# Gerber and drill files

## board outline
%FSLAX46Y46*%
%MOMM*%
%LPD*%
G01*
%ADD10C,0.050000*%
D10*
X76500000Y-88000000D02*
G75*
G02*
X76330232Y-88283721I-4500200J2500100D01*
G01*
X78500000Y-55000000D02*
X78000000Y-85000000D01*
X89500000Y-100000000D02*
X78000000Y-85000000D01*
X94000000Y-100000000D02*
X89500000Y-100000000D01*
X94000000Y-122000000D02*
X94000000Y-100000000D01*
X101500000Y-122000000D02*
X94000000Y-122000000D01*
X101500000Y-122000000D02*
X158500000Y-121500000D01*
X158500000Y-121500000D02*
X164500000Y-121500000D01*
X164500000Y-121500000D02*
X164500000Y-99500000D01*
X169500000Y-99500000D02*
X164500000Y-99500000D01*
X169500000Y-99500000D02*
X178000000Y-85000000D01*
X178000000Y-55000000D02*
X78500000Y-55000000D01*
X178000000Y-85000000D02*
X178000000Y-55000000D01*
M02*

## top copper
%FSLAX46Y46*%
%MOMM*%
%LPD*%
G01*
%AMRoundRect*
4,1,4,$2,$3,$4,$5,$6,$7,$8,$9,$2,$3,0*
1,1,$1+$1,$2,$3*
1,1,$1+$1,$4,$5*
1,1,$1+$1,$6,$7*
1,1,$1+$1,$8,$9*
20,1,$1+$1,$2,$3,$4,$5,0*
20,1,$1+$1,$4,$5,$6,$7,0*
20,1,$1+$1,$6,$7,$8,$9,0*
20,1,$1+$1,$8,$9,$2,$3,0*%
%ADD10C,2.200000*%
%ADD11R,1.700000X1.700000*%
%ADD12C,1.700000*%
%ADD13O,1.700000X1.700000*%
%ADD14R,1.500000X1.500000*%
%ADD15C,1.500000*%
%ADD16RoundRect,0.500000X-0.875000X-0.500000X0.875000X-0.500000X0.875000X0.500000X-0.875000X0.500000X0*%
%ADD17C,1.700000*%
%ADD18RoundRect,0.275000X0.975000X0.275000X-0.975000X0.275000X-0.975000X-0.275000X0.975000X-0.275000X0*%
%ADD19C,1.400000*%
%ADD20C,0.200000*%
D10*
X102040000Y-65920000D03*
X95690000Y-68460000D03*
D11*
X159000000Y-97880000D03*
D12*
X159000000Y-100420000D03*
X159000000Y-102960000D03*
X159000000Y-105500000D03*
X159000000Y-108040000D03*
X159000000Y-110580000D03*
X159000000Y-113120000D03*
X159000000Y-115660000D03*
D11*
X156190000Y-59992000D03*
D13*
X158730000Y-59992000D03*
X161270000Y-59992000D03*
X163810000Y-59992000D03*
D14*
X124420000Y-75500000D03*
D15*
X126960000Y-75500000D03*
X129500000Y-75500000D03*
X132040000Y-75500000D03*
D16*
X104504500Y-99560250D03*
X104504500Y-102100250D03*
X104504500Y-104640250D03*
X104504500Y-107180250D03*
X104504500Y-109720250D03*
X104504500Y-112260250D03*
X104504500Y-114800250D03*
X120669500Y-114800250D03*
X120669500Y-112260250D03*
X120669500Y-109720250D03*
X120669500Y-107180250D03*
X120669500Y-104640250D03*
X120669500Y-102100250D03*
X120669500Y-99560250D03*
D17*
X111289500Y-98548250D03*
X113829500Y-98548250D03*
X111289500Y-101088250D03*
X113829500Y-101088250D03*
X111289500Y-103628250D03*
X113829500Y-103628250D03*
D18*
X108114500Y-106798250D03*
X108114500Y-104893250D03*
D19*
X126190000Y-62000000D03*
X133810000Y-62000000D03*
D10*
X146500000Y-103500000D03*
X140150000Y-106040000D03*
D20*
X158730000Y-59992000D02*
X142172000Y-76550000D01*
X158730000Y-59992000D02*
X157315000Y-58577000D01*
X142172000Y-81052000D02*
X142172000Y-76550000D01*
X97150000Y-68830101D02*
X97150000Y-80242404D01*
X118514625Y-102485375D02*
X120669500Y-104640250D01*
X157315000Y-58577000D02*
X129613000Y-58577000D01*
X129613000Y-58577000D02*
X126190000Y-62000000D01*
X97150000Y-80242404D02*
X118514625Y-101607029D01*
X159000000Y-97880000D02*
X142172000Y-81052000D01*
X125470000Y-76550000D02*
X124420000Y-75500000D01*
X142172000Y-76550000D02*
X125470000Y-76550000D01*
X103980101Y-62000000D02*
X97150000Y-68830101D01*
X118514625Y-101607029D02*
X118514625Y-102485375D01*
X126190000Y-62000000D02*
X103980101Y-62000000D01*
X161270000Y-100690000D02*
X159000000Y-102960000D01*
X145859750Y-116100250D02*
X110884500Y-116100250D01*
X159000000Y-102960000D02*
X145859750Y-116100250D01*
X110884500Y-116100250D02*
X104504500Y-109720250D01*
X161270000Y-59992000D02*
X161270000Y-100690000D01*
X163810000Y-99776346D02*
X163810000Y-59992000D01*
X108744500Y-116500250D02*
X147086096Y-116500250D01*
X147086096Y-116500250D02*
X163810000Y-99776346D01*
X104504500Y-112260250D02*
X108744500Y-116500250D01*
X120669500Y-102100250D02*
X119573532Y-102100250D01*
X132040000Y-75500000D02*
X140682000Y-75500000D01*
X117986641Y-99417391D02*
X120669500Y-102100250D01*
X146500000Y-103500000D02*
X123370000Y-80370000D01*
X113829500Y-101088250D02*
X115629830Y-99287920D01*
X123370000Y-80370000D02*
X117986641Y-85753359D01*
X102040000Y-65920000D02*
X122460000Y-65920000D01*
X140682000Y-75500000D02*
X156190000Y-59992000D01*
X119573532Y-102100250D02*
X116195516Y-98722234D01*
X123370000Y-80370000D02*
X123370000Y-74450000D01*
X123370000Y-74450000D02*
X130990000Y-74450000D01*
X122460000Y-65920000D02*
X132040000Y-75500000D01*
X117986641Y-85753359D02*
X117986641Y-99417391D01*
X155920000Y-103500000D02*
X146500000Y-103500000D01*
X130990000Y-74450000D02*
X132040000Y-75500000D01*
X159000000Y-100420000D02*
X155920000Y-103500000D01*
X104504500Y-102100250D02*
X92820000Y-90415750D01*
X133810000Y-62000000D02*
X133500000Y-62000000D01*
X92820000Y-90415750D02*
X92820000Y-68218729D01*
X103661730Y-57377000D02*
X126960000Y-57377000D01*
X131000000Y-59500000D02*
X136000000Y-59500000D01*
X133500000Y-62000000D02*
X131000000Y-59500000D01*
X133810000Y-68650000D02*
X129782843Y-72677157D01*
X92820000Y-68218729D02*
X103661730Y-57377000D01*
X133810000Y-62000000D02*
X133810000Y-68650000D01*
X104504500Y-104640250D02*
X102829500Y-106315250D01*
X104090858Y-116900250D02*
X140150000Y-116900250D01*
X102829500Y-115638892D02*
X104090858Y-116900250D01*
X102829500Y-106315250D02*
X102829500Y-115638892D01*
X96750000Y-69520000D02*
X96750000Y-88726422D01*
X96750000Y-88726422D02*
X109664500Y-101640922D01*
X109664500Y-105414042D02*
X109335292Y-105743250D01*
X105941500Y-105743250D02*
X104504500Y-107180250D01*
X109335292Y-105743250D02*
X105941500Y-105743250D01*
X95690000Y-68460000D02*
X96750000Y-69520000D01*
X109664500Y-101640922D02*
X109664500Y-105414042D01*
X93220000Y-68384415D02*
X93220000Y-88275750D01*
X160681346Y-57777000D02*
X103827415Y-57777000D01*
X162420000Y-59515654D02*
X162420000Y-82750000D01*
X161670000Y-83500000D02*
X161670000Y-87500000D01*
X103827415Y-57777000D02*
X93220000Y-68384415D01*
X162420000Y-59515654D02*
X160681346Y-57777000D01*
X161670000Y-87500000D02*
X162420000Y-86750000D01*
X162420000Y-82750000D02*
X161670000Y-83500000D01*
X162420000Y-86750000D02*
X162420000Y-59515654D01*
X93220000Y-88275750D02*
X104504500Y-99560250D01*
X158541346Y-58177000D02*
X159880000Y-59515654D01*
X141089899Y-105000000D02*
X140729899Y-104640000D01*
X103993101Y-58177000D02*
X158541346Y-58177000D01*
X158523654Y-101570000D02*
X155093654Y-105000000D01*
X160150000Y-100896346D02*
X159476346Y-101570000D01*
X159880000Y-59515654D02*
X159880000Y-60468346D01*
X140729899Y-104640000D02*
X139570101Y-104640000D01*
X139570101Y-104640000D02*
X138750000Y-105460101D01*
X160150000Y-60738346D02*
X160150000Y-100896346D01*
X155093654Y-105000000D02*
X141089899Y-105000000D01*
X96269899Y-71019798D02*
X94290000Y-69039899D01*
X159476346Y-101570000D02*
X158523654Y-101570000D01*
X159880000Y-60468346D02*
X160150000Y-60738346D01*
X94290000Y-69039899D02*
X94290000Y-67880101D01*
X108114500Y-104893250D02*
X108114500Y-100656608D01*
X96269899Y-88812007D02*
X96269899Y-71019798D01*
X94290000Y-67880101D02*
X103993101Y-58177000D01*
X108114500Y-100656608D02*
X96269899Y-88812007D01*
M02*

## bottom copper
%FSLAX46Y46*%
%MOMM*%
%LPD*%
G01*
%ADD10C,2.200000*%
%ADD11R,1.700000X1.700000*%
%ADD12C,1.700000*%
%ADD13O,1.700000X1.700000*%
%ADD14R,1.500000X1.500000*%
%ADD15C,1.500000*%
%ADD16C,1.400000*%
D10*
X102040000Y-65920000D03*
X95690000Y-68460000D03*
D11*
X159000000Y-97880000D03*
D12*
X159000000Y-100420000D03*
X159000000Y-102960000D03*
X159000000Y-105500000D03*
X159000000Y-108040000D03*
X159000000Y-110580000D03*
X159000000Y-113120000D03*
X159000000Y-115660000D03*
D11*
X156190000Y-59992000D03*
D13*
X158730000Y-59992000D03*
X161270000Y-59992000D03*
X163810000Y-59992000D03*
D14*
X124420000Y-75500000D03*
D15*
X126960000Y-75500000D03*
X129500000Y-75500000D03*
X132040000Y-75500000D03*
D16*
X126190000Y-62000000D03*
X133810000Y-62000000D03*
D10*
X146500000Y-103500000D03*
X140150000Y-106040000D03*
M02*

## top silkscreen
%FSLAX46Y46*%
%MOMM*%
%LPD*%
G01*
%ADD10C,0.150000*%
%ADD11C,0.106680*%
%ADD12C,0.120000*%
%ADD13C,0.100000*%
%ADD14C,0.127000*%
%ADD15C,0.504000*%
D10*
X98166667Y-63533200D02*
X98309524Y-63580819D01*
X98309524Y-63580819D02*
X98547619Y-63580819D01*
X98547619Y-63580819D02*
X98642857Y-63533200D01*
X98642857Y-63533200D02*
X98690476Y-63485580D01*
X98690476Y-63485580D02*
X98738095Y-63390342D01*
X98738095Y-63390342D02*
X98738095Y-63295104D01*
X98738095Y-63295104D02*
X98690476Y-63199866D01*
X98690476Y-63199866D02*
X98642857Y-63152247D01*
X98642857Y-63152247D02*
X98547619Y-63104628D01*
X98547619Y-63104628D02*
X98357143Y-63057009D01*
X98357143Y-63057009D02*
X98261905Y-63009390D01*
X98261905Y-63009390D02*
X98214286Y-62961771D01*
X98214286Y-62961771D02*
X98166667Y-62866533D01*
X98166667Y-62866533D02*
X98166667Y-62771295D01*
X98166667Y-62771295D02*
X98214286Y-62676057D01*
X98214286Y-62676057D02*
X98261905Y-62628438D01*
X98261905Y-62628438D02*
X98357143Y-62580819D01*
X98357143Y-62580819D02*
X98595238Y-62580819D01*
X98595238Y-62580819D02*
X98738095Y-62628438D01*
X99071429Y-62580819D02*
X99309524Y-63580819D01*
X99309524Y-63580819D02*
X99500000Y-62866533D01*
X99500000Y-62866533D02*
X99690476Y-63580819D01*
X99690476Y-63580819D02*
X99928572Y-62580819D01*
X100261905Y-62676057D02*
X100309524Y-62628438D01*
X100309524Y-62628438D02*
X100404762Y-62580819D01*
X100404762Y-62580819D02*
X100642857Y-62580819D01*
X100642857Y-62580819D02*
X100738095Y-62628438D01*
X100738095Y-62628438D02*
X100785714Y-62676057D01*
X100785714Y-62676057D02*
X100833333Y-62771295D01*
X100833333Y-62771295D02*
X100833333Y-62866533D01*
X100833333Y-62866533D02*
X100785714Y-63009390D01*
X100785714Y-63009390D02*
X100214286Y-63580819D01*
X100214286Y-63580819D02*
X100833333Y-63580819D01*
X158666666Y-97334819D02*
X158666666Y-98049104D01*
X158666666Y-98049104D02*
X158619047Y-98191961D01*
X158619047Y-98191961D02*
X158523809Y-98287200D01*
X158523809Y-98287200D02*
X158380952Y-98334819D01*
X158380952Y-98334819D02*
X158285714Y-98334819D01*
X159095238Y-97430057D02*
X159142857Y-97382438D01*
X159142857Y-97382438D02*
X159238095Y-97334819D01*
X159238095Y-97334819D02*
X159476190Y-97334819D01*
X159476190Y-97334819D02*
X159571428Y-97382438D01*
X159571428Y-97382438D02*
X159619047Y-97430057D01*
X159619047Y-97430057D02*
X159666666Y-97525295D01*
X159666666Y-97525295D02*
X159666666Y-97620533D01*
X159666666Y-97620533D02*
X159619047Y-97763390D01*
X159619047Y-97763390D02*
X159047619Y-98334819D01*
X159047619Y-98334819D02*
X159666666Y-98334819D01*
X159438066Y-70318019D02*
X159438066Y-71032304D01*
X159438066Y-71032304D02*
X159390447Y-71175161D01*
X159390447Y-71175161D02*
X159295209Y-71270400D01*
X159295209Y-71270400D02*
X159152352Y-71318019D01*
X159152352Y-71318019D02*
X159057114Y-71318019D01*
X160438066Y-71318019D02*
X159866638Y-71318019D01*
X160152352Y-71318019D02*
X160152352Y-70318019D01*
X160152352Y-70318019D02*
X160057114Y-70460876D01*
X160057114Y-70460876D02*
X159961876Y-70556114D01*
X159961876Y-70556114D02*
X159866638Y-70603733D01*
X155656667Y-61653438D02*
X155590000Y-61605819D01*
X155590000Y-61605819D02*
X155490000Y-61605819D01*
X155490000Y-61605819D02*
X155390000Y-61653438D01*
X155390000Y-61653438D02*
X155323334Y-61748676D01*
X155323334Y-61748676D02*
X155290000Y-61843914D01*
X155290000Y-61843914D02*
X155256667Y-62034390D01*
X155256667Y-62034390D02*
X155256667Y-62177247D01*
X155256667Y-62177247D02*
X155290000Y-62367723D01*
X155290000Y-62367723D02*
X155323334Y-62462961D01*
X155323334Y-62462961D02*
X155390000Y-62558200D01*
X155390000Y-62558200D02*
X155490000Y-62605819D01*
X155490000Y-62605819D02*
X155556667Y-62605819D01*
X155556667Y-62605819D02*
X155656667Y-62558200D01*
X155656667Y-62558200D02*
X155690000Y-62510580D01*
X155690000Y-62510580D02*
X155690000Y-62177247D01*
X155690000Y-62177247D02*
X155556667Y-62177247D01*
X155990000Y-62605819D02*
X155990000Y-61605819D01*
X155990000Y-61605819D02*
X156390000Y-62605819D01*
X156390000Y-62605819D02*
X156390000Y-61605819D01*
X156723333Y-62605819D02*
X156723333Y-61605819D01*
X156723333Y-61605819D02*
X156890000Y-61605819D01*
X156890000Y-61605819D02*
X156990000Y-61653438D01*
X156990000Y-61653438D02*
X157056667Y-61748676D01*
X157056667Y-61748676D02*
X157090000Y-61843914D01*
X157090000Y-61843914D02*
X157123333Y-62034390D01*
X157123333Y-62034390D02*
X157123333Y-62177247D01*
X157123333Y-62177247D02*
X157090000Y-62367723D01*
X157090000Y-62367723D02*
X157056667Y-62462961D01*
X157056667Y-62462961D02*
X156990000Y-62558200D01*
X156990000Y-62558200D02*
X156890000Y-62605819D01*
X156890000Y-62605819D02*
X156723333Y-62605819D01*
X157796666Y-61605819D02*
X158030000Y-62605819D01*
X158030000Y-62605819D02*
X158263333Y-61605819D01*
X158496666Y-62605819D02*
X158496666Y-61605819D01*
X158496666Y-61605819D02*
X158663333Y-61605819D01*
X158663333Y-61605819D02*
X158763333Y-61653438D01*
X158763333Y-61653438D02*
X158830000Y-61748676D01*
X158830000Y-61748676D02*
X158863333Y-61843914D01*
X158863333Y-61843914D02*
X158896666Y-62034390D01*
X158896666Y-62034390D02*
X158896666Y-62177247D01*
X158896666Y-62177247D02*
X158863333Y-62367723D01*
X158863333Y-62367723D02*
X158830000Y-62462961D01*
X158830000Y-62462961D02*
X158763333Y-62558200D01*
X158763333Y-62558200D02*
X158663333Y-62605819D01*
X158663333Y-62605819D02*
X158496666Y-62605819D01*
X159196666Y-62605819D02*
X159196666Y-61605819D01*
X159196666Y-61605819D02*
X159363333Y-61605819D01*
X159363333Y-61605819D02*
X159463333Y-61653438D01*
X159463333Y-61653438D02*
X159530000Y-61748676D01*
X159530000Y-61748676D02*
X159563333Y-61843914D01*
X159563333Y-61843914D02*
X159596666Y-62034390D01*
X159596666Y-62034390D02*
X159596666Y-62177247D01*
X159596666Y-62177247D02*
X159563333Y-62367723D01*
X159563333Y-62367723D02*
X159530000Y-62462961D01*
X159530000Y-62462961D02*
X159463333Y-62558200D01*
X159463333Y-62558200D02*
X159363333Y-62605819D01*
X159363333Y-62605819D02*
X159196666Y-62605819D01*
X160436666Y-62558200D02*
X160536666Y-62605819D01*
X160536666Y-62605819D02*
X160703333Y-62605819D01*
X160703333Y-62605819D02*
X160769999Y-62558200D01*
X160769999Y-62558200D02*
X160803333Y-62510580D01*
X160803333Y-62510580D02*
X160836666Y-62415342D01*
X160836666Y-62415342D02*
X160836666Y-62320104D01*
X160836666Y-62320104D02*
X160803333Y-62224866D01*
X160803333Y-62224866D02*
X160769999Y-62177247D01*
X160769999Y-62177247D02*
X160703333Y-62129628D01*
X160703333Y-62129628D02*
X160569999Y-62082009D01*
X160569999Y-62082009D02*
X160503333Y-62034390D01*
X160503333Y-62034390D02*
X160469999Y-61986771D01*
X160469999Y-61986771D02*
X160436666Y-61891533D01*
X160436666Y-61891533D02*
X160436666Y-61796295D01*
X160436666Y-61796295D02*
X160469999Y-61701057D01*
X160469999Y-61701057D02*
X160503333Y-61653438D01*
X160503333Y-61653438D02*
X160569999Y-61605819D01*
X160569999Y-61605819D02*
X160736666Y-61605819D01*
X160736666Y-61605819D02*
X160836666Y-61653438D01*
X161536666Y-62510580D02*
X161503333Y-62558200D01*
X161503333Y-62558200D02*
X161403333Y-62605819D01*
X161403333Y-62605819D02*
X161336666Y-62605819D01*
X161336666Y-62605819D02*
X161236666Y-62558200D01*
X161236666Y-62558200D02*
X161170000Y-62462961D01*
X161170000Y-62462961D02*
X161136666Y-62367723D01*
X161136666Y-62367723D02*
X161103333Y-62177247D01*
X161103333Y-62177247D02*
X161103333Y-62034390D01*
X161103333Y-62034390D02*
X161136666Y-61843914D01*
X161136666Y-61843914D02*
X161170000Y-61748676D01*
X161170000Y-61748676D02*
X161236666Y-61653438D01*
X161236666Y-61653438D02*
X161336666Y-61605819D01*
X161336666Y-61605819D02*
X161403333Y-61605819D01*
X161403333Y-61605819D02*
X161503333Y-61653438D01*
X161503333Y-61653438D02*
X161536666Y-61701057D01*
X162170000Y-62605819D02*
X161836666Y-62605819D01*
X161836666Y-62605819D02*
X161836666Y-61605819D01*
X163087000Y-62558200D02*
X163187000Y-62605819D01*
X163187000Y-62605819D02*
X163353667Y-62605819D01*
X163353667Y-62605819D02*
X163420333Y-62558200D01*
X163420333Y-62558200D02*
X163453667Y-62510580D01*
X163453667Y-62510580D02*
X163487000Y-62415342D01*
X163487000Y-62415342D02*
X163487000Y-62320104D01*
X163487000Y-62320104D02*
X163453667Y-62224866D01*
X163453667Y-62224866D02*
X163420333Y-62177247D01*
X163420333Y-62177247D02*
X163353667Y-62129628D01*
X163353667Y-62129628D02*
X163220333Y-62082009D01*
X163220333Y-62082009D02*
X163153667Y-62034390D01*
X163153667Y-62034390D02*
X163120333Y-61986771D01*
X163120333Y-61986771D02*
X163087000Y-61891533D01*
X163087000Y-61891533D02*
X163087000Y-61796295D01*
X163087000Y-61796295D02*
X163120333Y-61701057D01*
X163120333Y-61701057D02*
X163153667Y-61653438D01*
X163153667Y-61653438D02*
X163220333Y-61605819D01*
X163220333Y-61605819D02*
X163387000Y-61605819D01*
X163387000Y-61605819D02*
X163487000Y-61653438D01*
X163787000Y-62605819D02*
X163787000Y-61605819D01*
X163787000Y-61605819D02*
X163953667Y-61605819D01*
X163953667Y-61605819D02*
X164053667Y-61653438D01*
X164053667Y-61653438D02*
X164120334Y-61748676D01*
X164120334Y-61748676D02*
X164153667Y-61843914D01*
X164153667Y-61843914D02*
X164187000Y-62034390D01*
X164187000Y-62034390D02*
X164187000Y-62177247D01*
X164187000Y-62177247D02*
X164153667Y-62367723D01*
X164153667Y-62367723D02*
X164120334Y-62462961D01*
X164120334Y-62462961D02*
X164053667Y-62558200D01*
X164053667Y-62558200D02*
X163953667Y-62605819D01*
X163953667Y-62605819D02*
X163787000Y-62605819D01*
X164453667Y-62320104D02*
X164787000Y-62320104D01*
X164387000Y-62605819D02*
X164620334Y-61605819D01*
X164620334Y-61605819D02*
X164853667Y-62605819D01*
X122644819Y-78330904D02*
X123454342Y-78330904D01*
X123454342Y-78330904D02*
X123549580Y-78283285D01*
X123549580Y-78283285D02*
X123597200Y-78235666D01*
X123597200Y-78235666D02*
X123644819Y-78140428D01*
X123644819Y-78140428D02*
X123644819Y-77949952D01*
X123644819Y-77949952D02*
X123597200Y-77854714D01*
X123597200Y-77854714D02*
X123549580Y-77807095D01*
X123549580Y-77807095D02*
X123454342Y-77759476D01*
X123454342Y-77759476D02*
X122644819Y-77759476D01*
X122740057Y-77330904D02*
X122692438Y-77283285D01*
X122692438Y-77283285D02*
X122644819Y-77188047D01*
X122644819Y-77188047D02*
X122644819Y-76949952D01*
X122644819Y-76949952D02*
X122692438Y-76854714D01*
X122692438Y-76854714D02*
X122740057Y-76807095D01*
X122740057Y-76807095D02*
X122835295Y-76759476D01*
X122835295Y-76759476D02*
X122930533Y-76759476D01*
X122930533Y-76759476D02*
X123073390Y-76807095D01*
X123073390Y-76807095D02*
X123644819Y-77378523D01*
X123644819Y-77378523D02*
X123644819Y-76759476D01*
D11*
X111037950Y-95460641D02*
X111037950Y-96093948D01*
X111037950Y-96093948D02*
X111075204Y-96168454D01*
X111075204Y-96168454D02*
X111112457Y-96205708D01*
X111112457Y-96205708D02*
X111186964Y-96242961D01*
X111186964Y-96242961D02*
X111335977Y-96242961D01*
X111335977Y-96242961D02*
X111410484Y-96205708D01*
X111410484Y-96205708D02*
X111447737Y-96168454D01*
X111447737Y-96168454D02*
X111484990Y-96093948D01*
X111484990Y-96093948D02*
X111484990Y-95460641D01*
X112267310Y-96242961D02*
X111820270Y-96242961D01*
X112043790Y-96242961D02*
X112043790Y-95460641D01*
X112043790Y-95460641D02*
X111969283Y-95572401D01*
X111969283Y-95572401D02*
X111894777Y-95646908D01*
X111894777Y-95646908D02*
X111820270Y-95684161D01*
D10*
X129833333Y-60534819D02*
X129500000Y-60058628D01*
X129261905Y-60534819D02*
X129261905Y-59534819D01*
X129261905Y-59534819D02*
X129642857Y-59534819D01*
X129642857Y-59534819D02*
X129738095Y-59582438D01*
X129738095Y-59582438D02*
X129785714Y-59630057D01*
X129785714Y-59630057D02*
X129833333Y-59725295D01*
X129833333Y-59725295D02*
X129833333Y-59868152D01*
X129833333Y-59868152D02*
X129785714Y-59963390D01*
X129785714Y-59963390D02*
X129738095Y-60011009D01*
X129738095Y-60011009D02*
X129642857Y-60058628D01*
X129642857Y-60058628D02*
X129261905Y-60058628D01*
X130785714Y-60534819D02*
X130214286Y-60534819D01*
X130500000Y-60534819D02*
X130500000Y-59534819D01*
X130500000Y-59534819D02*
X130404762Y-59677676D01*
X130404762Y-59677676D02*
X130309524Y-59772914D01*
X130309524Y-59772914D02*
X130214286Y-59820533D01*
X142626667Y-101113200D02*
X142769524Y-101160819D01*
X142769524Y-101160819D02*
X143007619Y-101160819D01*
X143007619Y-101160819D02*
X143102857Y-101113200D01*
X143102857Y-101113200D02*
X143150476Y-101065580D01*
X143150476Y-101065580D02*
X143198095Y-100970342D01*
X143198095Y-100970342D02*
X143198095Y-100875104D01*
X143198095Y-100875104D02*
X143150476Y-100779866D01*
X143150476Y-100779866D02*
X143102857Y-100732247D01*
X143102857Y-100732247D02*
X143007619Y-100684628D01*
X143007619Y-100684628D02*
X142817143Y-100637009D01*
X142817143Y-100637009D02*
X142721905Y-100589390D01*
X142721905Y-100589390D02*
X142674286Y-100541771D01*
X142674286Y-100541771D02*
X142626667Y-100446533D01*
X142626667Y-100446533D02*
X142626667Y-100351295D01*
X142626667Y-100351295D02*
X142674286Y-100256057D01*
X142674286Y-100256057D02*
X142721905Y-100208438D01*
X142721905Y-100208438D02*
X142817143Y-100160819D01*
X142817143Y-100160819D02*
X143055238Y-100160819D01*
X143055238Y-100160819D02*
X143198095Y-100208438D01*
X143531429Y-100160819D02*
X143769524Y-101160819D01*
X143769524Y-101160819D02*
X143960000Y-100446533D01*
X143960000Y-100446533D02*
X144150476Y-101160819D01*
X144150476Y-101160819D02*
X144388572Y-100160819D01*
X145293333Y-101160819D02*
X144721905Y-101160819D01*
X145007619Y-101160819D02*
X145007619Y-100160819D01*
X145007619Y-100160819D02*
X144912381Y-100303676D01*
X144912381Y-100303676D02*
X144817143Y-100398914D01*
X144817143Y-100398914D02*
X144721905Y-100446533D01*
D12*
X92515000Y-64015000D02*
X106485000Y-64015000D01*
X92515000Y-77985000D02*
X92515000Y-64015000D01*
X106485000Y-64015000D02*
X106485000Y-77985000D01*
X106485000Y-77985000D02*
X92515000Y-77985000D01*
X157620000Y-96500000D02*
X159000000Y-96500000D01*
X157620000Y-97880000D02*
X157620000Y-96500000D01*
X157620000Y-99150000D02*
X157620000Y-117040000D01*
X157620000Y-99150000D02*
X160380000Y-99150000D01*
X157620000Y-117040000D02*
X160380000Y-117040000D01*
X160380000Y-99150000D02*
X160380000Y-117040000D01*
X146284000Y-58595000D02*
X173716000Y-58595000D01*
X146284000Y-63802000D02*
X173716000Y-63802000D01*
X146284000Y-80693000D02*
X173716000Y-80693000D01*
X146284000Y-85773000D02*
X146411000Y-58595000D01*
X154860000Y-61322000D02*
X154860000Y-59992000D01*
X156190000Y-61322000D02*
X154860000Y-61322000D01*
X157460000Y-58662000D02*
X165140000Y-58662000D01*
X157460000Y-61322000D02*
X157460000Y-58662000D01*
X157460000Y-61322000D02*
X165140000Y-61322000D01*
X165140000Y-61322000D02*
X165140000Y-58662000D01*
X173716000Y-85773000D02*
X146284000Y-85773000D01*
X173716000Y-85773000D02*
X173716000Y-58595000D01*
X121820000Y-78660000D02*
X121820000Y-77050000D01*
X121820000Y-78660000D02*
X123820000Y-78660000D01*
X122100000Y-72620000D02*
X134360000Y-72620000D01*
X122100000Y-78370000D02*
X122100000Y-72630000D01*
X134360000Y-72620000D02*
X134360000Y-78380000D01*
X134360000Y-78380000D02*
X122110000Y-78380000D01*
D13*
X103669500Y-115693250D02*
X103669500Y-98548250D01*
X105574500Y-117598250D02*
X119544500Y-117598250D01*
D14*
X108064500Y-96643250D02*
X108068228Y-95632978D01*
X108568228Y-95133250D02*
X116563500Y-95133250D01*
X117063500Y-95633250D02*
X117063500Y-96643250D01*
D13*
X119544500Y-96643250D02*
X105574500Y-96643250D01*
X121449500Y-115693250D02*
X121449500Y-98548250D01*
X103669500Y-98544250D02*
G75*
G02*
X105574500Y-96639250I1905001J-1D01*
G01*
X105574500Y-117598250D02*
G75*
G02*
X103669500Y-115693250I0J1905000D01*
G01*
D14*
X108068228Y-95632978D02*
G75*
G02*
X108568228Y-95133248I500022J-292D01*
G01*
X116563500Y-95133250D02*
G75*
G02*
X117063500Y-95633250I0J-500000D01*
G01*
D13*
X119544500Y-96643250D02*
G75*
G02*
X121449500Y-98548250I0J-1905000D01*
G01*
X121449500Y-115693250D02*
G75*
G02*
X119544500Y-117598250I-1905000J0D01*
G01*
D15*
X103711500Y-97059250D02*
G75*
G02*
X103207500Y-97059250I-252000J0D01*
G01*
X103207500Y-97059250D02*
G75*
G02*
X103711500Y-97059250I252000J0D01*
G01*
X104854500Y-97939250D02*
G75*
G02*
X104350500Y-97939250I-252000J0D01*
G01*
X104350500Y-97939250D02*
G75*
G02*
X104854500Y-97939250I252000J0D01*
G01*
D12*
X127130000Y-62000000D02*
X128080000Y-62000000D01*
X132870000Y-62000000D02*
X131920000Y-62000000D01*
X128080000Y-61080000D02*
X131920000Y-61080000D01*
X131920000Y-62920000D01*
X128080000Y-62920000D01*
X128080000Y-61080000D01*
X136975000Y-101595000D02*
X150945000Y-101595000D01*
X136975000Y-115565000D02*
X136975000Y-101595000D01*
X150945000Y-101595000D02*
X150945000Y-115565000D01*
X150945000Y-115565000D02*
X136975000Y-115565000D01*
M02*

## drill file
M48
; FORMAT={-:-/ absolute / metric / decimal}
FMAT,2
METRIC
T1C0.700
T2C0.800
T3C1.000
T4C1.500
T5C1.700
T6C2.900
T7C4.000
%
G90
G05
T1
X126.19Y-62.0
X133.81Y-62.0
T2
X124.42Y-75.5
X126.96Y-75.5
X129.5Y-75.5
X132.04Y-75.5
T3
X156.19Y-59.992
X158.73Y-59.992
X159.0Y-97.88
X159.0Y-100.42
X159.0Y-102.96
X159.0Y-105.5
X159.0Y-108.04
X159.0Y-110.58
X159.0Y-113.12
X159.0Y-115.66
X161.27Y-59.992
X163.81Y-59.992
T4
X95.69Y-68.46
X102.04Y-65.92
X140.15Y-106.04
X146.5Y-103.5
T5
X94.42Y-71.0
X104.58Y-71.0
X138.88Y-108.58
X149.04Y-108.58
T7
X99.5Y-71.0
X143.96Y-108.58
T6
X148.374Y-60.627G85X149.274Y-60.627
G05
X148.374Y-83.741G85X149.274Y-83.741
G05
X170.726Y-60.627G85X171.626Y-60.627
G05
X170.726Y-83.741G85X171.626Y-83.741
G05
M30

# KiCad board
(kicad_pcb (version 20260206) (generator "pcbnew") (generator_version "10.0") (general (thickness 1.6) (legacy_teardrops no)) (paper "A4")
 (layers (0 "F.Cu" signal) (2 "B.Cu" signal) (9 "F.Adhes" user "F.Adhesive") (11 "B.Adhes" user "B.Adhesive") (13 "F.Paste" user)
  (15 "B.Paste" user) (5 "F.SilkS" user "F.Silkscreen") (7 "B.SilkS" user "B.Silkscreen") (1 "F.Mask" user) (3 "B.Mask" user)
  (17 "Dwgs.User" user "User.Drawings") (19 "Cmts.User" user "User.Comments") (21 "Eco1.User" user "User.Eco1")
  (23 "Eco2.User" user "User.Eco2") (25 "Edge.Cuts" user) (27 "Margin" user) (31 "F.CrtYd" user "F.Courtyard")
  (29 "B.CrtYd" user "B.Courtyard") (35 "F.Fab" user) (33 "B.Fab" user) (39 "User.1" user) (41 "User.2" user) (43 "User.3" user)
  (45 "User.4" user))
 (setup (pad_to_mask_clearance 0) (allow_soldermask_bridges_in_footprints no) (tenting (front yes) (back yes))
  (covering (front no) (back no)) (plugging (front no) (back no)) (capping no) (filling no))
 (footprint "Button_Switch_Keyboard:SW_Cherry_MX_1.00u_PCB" (layer "F.Cu") (at 102.04 65.92)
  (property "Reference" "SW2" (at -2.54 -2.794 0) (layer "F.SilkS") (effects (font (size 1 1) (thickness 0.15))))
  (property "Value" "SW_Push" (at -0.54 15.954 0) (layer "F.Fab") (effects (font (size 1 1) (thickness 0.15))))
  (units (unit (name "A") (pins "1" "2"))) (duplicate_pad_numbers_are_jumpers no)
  (fp_line (start -9.525 -1.905) (end 4.445 -1.905) (stroke (width 0.12) (type solid)) (layer "F.SilkS"))
  (fp_line (start -9.525 12.065) (end -9.525 -1.905) (stroke (width 0.12) (type solid)) (layer "F.SilkS"))
  (fp_line (start 4.445 -1.905) (end 4.445 12.065) (stroke (width 0.12) (type solid)) (layer "F.SilkS"))
  (fp_line (start 4.445 12.065) (end -9.525 12.065) (stroke (width 0.12) (type solid)) (layer "F.SilkS"))
  (pad "" np_thru_hole circle (at -7.62 5.08) (size 1.7 1.7) (drill 1.7) (layers "*.Cu" "*.Mask"))
  (pad "" np_thru_hole circle (at -2.54 5.08) (size 4 4) (drill 4) (layers "*.Cu" "*.Mask"))
  (pad "" np_thru_hole circle (at 2.54 5.08) (size 1.7 1.7) (drill 1.7) (layers "*.Cu" "*.Mask"))
  (pad "1" thru_hole circle (at 0 0) (size 2.2 2.2) (drill 1.5) (layers "*.Cu" "*.Mask") (remove_unused_layers no) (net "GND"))
  (pad "2" thru_hole circle (at -6.35 2.54) (size 2.2 2.2) (drill 1.5) (layers "*.Cu" "*.Mask") (remove_unused_layers no) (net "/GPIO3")))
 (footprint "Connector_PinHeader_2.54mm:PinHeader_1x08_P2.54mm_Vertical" (layer "F.Cu") (at 159 97.88)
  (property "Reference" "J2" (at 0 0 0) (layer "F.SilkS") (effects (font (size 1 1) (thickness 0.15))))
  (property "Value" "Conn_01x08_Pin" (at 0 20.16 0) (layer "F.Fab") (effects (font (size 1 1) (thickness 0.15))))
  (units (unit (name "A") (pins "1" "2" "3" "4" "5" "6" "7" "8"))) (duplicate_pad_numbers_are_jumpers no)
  (fp_line (start -1.38 -1.38) (end 0 -1.38) (stroke (width 0.12) (type solid)) (layer "F.SilkS"))
  (fp_line (start -1.38 0) (end -1.38 -1.38) (stroke (width 0.12) (type solid)) (layer "F.SilkS"))
  (fp_line (start -1.38 1.27) (end -1.38 19.16) (stroke (width 0.12) (type solid)) (layer "F.SilkS"))
  (fp_line (start -1.38 1.27) (end 1.38 1.27) (stroke (width 0.12) (type solid)) (layer "F.SilkS"))
  (fp_line (start -1.38 19.16) (end 1.38 19.16) (stroke (width 0.12) (type solid)) (layer "F.SilkS"))
  (fp_line (start 1.38 1.27) (end 1.38 19.16) (stroke (width 0.12) (type solid)) (layer "F.SilkS"))
  (pad "1" thru_hole rect (at 0 0) (size 1.7 1.7) (drill 1) (layers "*.Cu" "*.Mask") (remove_unused_layers no) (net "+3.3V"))
  (pad "2" thru_hole circle (at 0 2.54) (size 1.7 1.7) (drill 1) (layers "*.Cu" "*.Mask") (remove_unused_layers no) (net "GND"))
  (pad "3" thru_hole circle (at 0 5.08) (size 1.7 1.7) (drill 1) (layers "*.Cu" "*.Mask") (remove_unused_layers no) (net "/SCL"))
  (pad "4" thru_hole circle (at 0 7.62) (size 1.7 1.7) (drill 1) (layers "*.Cu" "*.Mask") (remove_unused_layers no) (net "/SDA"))
  (pad "5" thru_hole circle (at 0 10.16) (size 1.7 1.7) (drill 1) (layers "*.Cu" "*.Mask") (remove_unused_layers no)
   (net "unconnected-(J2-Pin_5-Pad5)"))
  (pad "6" thru_hole circle (at 0 12.7) (size 1.7 1.7) (drill 1) (layers "*.Cu" "*.Mask") (remove_unused_layers no)
   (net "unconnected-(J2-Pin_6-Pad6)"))
  (pad "7" thru_hole circle (at 0 15.24) (size 1.7 1.7) (drill 1) (layers "*.Cu" "*.Mask") (remove_unused_layers no)
   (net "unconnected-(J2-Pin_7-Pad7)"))
  (pad "8" thru_hole circle (at 0 17.78) (size 1.7 1.7) (drill 1) (layers "*.Cu" "*.Mask") (remove_unused_layers no)
   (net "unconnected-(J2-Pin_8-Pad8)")))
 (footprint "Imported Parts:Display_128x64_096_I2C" (layer "F.Cu") (at 160 59.992)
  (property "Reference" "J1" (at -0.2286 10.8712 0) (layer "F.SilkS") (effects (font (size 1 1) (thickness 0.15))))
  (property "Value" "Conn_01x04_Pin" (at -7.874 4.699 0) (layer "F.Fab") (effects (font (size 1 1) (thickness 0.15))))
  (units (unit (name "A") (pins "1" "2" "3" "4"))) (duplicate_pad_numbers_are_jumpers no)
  (fp_line (start -13.716 -1.397) (end 13.716 -1.397) (stroke (width 0.12) (type solid)) (layer "F.SilkS"))
  (fp_line (start -13.716 3.81) (end 13.716 3.81) (stroke (width 0.12) (type solid)) (layer "F.SilkS"))
  (fp_line (start -13.716 20.701) (end 13.716 20.701) (stroke (width 0.12) (type solid)) (layer "F.SilkS"))
  (fp_line (start -13.716 25.781) (end -13.589 -1.397) (stroke (width 0.12) (type solid)) (layer "F.SilkS"))
  (fp_line (start -5.14 1.33) (end -5.14 0) (stroke (width 0.12) (type solid)) (layer "F.SilkS"))
  (fp_line (start -3.81 1.33) (end -5.14 1.33) (stroke (width 0.12) (type solid)) (layer "F.SilkS"))
  (fp_line (start -2.54 -1.33) (end 5.14 -1.33) (stroke (width 0.12) (type solid)) (layer "F.SilkS"))
  (fp_line (start -2.54 1.33) (end -2.54 -1.33) (stroke (width 0.12) (type solid)) (layer "F.SilkS"))
  (fp_line (start -2.54 1.33) (end 5.14 1.33) (stroke (width 0.12) (type solid)) (layer "F.SilkS"))
  (fp_line (start 5.14 1.33) (end 5.14 -1.33) (stroke (width 0.12) (type solid)) (layer "F.SilkS"))
  (fp_line (start 13.716 25.781) (end -13.716 25.781) (stroke (width 0.12) (type solid)) (layer "F.SilkS"))
  (fp_line (start 13.716 25.781) (end 13.716 -1.397) (stroke (width 0.12) (type solid)) (layer "F.SilkS"))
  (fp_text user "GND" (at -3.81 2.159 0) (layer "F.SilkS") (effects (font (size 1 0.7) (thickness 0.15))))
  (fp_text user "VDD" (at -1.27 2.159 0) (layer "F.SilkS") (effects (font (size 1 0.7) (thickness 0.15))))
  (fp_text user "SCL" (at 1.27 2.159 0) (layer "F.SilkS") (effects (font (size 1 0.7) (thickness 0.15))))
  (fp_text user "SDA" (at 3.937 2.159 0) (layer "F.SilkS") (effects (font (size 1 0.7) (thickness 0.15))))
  (pad "" np_thru_hole oval (at -11.176 0.635) (size 3.8 2.9) (drill oval 3.8 2.9) (layers "*.Cu" "*.Mask"))
  (pad "" np_thru_hole oval (at -11.176 23.749) (size 3.8 2.9) (drill oval 3.8 2.9) (layers "*.Cu" "*.Mask"))
  (pad "" np_thru_hole oval (at 11.176 0.635) (size 3.8 2.9) (drill oval 3.8 2.9) (layers "*.Cu" "*.Mask"))
  (pad "" np_thru_hole oval (at 11.176 23.749) (size 3.8 2.9) (drill oval 3.8 2.9) (layers "*.Cu" "*.Mask"))
  (pad "1" thru_hole rect (at -3.81 0 90) (size 1.7 1.7) (drill 1) (layers "*.Cu" "*.Mask") (remove_unused_layers no) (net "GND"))
  (pad "2" thru_hole oval (at -1.27 0 90) (size 1.7 1.7) (drill 1) (layers "*.Cu" "*.Mask") (remove_unused_layers no) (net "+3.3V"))
  (pad "3" thru_hole oval (at 1.27 0 90) (size 1.7 1.7) (drill 1) (layers "*.Cu" "*.Mask") (remove_unused_layers no) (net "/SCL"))
  (pad "4" thru_hole oval (at 3.81 0 90) (size 1.7 1.7) (drill 1) (layers "*.Cu" "*.Mask") (remove_unused_layers no) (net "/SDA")))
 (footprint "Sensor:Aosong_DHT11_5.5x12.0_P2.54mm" (layer "F.Cu") (at 124.42 75.5 90)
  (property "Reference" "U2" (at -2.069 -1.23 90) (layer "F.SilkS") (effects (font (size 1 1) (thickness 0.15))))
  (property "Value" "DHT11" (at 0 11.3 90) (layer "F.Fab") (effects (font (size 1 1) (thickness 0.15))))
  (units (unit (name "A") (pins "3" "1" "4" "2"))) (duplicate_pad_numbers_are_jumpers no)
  (fp_line (start -3.16 -2.6) (end -1.55 -2.6) (stroke (width 0.12) (type solid)) (layer "F.SilkS"))
  (fp_line (start -3.16 -2.6) (end -3.16 -0.6) (stroke (width 0.12) (type solid)) (layer "F.SilkS"))
  (fp_line (start 2.88 -2.32) (end 2.88 9.94) (stroke (width 0.12) (type solid)) (layer "F.SilkS"))
  (fp_line (start -2.87 -2.32) (end 2.87 -2.32) (stroke (width 0.12) (type solid)) (layer "F.SilkS"))
  (fp_line (start 2.88 9.94) (end -2.88 9.94) (stroke (width 0.12) (type solid)) (layer "F.SilkS"))
  (fp_line (start -2.88 9.94) (end -2.88 -2.31) (stroke (width 0.12) (type solid)) (layer "F.SilkS"))
  (pad "1" thru_hole rect (at 0 0 90) (size 1.5 1.5) (drill 0.8) (layers "*.Cu" "*.Mask") (remove_unused_layers no) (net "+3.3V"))
  (pad "2" thru_hole circle (at 0 2.54 90) (size 1.5 1.5) (drill 0.8) (layers "*.Cu" "*.Mask") (remove_unused_layers no) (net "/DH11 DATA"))
  (pad "3" thru_hole circle (at 0 5.08 90) (size 1.5 1.5) (drill 0.8) (layers "*.Cu" "*.Mask") (remove_unused_layers no)
   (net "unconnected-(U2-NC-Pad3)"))
  (pad "4" thru_hole circle (at 0 7.62 90) (size 1.5 1.5) (drill 0.8) (layers "*.Cu" "*.Mask") (remove_unused_layers no) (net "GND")))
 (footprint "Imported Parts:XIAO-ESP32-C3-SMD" (layer "F.Cu") (at 103.6695 117.68025)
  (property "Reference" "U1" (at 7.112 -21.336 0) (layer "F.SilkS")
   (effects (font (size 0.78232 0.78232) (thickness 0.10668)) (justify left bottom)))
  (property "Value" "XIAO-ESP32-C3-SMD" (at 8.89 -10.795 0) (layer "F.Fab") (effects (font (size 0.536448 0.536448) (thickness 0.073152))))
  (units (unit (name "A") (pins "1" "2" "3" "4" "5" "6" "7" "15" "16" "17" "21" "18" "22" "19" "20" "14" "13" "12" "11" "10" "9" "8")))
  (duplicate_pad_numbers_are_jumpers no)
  (fp_line (start 0 -1.987) (end 0 -19.132) (stroke (width 0.1) (type solid)) (layer "F.SilkS"))
  (fp_line (start 1.905 -0.082) (end 15.875 -0.082) (stroke (width 0.1) (type solid)) (layer "F.SilkS"))
  (fp_line (start 4.395 -21.037) (end 4.398728 -22.047272) (stroke (width 0.127) (type solid)) (layer "F.SilkS"))
  (fp_line (start 4.898728 -22.547) (end 12.894 -22.547) (stroke (width 0.127) (type solid)) (layer "F.SilkS"))
  (fp_line (start 13.394 -22.047) (end 13.394 -21.037) (stroke (width 0.127) (type solid)) (layer "F.SilkS"))
  (fp_line (start 15.875 -21.037) (end 1.905 -21.037) (stroke (width 0.1) (type solid)) (layer "F.SilkS"))
  (fp_line (start 17.78 -1.987) (end 17.78 -19.132) (stroke (width 0.1) (type solid)) (layer "F.SilkS"))
  (fp_arc (start 0 -19.136) (mid 0.557962 -20.483038) (end 1.905 -21.041) (stroke (width 0.1) (type solid)) (layer "F.SilkS"))
  (fp_arc (start 1.905 -0.082) (mid 0.557962 -0.639962) (end 0 -1.987) (stroke (width 0.1) (type solid)) (layer "F.SilkS"))
  (fp_arc (start 4.398728 -22.047272) (mid 4.545272 -22.40064) (end 4.898728 -22.547) (stroke (width 0.127) (type default))
   (layer "F.SilkS"))
  (fp_arc (start 12.894 -22.547) (mid 13.247553 -22.400553) (end 13.394 -22.047) (stroke (width 0.127) (type default)) (layer "F.SilkS"))
  (fp_arc (start 15.875 -21.037) (mid 17.222038 -20.479038) (end 17.78 -19.132) (stroke (width 0.1) (type solid)) (layer "F.SilkS"))
  (fp_arc (start 17.78 -1.987) (mid 17.222038 -0.639962) (end 15.875 -0.082) (stroke (width 0.1) (type solid)) (layer "F.SilkS"))
  (fp_circle (center -0.21 -20.621) (end -0.21 -20.875) (stroke (width 0.5) (type solid)) (fill yes) (layer "F.SilkS"))
  (fp_circle (center 0.933 -19.741) (end 0.933 -19.995) (stroke (width 0.5) (type solid)) (fill yes) (layer "F.SilkS"))
  (pad "1" smd roundrect (at 0.835 -18.12) (size 2.75 2) (layers "F.Cu" "F.Mask" "F.Paste") (roundrect_rratio 0.25)
   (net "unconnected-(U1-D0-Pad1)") (solder_mask_margin 0.0508) (thermal_bridge_angle 45))
  (pad "2" smd roundrect (at 0.835 -15.58) (size 2.75 2) (layers "F.Cu" "F.Mask" "F.Paste") (roundrect_rratio 0.25) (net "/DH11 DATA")
   (solder_mask_margin 0.0508) (thermal_bridge_angle 45))
  (pad "3" smd roundrect (at 0.835 -13.04) (size 2.75 2) (layers "F.Cu" "F.Mask" "F.Paste") (roundrect_rratio 0.25) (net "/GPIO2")
   (solder_mask_margin 0.0508) (thermal_bridge_angle 45))
  (pad "4" smd roundrect (at 0.835 -10.5) (size 2.75 2) (layers "F.Cu" "F.Mask" "F.Paste") (roundrect_rratio 0.25) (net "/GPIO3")
   (solder_mask_margin 0.0508) (thermal_bridge_angle 45))
  (pad "5" smd roundrect (at 0.835 -7.96) (size 2.75 2) (layers "F.Cu" "F.Mask" "F.Paste") (roundrect_rratio 0.25) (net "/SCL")
   (solder_mask_margin 0.0508) (thermal_bridge_angle 45))
  (pad "6" smd roundrect (at 0.835 -5.42) (size 2.75 2) (layers "F.Cu" "F.Mask" "F.Paste") (roundrect_rratio 0.25) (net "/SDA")
   (solder_mask_margin 0.0508) (thermal_bridge_angle 45))
  (pad "7" smd roundrect (at 0.835 -2.88) (size 2.75 2) (layers "F.Cu" "F.Mask" "F.Paste") (roundrect_rratio 0.25)
   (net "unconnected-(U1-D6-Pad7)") (solder_mask_margin 0.0508) (thermal_bridge_angle 45))
  (pad "8" smd roundrect (at 17 -2.88) (size 2.75 2) (layers "F.Cu" "F.Mask" "F.Paste") (roundrect_rratio 0.25)
   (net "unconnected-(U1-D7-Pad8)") (solder_mask_margin 0.0508) (thermal_bridge_angle 45))
  (pad "9" smd roundrect (at 17 -5.42) (size 2.75 2) (layers "F.Cu" "F.Mask" "F.Paste") (roundrect_rratio 0.25)
   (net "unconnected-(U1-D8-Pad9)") (solder_mask_margin 0.0508) (thermal_bridge_angle 45))
  (pad "10" smd roundrect (at 17 -7.96) (size 2.75 2) (layers "F.Cu" "F.Mask" "F.Paste") (roundrect_rratio 0.25)
   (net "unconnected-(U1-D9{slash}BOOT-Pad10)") (solder_mask_margin 0.0508) (thermal_bridge_angle 45))
  (pad "11" smd roundrect (at 17 -10.5) (size 2.75 2) (layers "F.Cu" "F.Mask" "F.Paste") (roundrect_rratio 0.25)
   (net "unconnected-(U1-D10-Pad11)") (solder_mask_margin 0.0508) (thermal_bridge_angle 45))
  (pad "12" smd roundrect (at 17 -13.04) (size 2.75 2) (layers "F.Cu" "F.Mask" "F.Paste") (roundrect_rratio 0.25) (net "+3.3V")
   (solder_mask_margin 0.0508) (thermal_bridge_angle 45))
  (pad "13" smd roundrect (at 17 -15.58) (size 2.75 2) (layers "F.Cu" "F.Mask" "F.Paste") (roundrect_rratio 0.25) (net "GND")
   (solder_mask_margin 0.0508) (thermal_bridge_angle 45))
  (pad "14" smd roundrect (at 17 -18.12) (size 2.75 2) (layers "F.Cu" "F.Mask" "F.Paste") (roundrect_rratio 0.25) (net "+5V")
   (solder_mask_margin 0.0508) (thermal_bridge_angle 45))
  (pad "15" smd circle (at 7.62 -19.132) (size 1.7 1.7) (layers "F.Cu" "F.Mask" "F.Paste") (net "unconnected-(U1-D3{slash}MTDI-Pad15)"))
  (pad "16" smd circle (at 10.16 -19.132) (size 1.7 1.7) (layers "F.Cu" "F.Mask" "F.Paste") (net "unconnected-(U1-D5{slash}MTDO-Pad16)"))
  (pad "17" smd circle (at 7.62 -16.592) (size 1.7 1.7) (layers "F.Cu" "F.Mask" "F.Paste") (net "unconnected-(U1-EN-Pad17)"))
  (pad "18" smd circle (at 10.16 -16.592) (size 1.7 1.7) (layers "F.Cu" "F.Mask" "F.Paste") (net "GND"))
  (pad "19" smd circle (at 7.62 -14.052) (size 1.7 1.7) (layers "F.Cu" "F.Mask" "F.Paste") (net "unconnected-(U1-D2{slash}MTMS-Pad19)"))
  (pad "20" smd circle (at 10.16 -14.052) (size 1.7 1.7) (layers "F.Cu" "F.Mask" "F.Paste") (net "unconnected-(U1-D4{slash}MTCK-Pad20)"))
  (pad "21" smd roundrect (at 4.445 -10.882 180) (size 2.5 1.1) (layers "F.Cu" "F.Mask" "F.Paste") (roundrect_rratio 0.25)
   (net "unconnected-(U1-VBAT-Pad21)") (thermal_bridge_angle 45))
  (pad "22" smd roundrect (at 4.445 -12.787 180) (size 2.5 1.1) (layers "F.Cu" "F.Mask" "F.Paste") (roundrect_rratio 0.25)
   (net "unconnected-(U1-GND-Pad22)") (thermal_bridge_angle 45)))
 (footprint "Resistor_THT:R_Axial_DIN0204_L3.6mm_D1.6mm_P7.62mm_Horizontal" (layer "F.Cu") (at 126.19 62)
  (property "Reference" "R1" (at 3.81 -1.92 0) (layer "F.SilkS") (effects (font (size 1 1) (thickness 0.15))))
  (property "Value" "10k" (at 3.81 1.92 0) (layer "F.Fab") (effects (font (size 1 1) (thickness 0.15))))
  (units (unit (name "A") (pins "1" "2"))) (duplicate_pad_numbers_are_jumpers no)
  (fp_line (start 0.94 0) (end 1.89 0) (stroke (width 0.12) (type solid)) (layer "F.SilkS"))
  (fp_line (start 6.68 0) (end 5.73 0) (stroke (width 0.12) (type solid)) (layer "F.SilkS"))
  (fp_rect (start 1.89 -0.92) (end 5.73 0.92) (stroke (width 0.12) (type solid)) (fill no) (layer "F.SilkS"))
  (pad "1" thru_hole circle (at 0 0) (size 1.4 1.4) (drill 0.7) (layers "*.Cu" "*.Mask") (remove_unused_layers no) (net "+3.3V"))
  (pad "2" thru_hole circle (at 7.62 0) (size 1.4 1.4) (drill 0.7) (layers "*.Cu" "*.Mask") (remove_unused_layers no) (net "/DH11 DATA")))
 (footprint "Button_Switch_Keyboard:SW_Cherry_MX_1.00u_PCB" (layer "F.Cu") (at 146.5 103.5)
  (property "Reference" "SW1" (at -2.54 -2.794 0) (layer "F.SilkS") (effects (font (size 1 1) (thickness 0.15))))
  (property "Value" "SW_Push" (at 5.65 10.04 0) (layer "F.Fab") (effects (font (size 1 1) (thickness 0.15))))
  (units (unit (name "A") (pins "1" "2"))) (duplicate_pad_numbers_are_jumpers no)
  (fp_line (start -9.525 -1.905) (end 4.445 -1.905) (stroke (width 0.12) (type solid)) (layer "F.SilkS"))
  (fp_line (start -9.525 12.065) (end -9.525 -1.905) (stroke (width 0.12) (type solid)) (layer "F.SilkS"))
  (fp_line (start 4.445 -1.905) (end 4.445 12.065) (stroke (width 0.12) (type solid)) (layer "F.SilkS"))
  (fp_line (start 4.445 12.065) (end -9.525 12.065) (stroke (width 0.12) (type solid)) (layer "F.SilkS"))
  (pad "" np_thru_hole circle (at -7.62 5.08) (size 1.7 1.7) (drill 1.7) (layers "*.Cu" "*.Mask"))
  (pad "" np_thru_hole circle (at -2.54 5.08) (size 4 4) (drill 4) (layers "*.Cu" "*.Mask"))
  (pad "" np_thru_hole circle (at 2.54 5.08) (size 1.7 1.7) (drill 1.7) (layers "*.Cu" "*.Mask"))
  (pad "1" thru_hole circle (at 0 0) (size 2.2 2.2) (drill 1.5) (layers "*.Cu" "*.Mask") (remove_unused_layers no) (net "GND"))
  (pad "2" thru_hole circle (at -6.35 2.54) (size 2.2 2.2) (drill 1.5) (layers "*.Cu" "*.Mask") (remove_unused_layers no) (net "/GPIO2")))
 (gr_arc (start 76.5 88) (mid 76.417394 88.143223) (end 76.330231 88.28372) (stroke (width 0.05) (type default)) (layer "Edge.Cuts"))
 (gr_line (start 78.5 55) (end 78 85) (stroke (width 0.05) (type default)) (layer "Edge.Cuts"))
 (gr_line (start 89.5 100) (end 78 85) (stroke (width 0.05) (type default)) (layer "Edge.Cuts"))
 (gr_line (start 94 100) (end 89.5 100) (stroke (width 0.05) (type default)) (layer "Edge.Cuts"))
 (gr_line (start 94 122) (end 94 100) (stroke (width 0.05) (type default)) (layer "Edge.Cuts"))
 (gr_line (start 101.5 122) (end 94 122) (stroke (width 0.05) (type default)) (layer "Edge.Cuts"))
 (gr_line (start 101.5 122) (end 158.5 121.5) (stroke (width 0.05) (type default)) (layer "Edge.Cuts"))
 (gr_line (start 158.5 121.5) (end 164.5 121.5) (stroke (width 0.05) (type default)) (layer "Edge.Cuts"))
 (gr_line (start 164.5 121.5) (end 164.5 99.5) (stroke (width 0.05) (type default)) (layer "Edge.Cuts"))
 (gr_line (start 169.5 99.5) (end 164.5 99.5) (stroke (width 0.05) (type default)) (layer "Edge.Cuts"))
 (gr_line (start 169.5 99.5) (end 178 85) (stroke (width 0.05) (type default)) (layer "Edge.Cuts"))
 (gr_line (start 178 55) (end 78.5 55) (stroke (width 0.05) (type default)) (layer "Edge.Cuts"))
 (gr_line (start 178 85) (end 178 55) (stroke (width 0.05) (type default)) (layer "Edge.Cuts"))
 (segment (start 158.73 59.992) (end 142.172 76.55) (width 0.2) (layer "F.Cu") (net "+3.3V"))
 (segment (start 158.73 59.992) (end 157.315 58.577) (width 0.2) (layer "F.Cu") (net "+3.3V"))
 (segment (start 142.172 81.052) (end 142.172 76.55) (width 0.2) (layer "F.Cu") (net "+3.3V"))
 (segment (start 97.15 68.830101) (end 97.15 80.242404) (width 0.2) (layer "F.Cu") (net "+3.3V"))
 (segment (start 118.514625 102.485375) (end 120.6695 104.64025) (width 0.2) (layer "F.Cu") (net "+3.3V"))
 (segment (start 157.315 58.577) (end 129.613 58.577) (width 0.2) (layer "F.Cu") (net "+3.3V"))
 (segment (start 129.613 58.577) (end 126.19 62) (width 0.2) (layer "F.Cu") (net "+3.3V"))
 (segment (start 97.15 80.242404) (end 118.514625 101.607029) (width 0.2) (layer "F.Cu") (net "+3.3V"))
 (segment (start 159 97.88) (end 142.172 81.052) (width 0.2) (layer "F.Cu") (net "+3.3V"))
 (segment (start 125.47 76.55) (end 124.42 75.5) (width 0.2) (layer "F.Cu") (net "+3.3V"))
 (segment (start 142.172 76.55) (end 125.47 76.55) (width 0.2) (layer "F.Cu") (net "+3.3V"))
 (segment (start 103.980101 62) (end 97.15 68.830101) (width 0.2) (layer "F.Cu") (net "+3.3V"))
 (segment (start 118.514625 101.607029) (end 118.514625 102.485375) (width 0.2) (layer "F.Cu") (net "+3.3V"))
 (segment (start 126.19 62) (end 103.980101 62) (width 0.2) (layer "F.Cu") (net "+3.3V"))
 (segment (start 161.27 100.69) (end 159 102.96) (width 0.2) (layer "F.Cu") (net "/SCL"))
 (segment (start 145.85975 116.10025) (end 110.8845 116.10025) (width 0.2) (layer "F.Cu") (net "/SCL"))
 (segment (start 159 102.96) (end 145.85975 116.10025) (width 0.2) (layer "F.Cu") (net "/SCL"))
 (segment (start 110.8845 116.10025) (end 104.5045 109.72025) (width 0.2) (layer "F.Cu") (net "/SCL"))
 (segment (start 161.27 59.992) (end 161.27 100.69) (width 0.2) (layer "F.Cu") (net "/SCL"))
 (segment (start 163.81 99.776346) (end 163.81 59.992) (width 0.2) (layer "F.Cu") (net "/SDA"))
 (segment (start 108.7445 116.50025) (end 147.086096 116.50025) (width 0.2) (layer "F.Cu") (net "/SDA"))
 (segment (start 147.086096 116.50025) (end 163.81 99.776346) (width 0.2) (layer "F.Cu") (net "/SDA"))
 (segment (start 104.5045 112.26025) (end 108.7445 116.50025) (width 0.2) (layer "F.Cu") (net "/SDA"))
 (segment (start 120.6695 102.10025) (end 119.573532 102.10025) (width 0.2) (layer "F.Cu") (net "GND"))
 (segment (start 132.04 75.5) (end 140.682 75.5) (width 0.2) (layer "F.Cu") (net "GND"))
 (segment (start 117.986641 99.417391) (end 120.6695 102.10025) (width 0.2) (layer "F.Cu") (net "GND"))
 (segment (start 146.5 103.5) (end 123.37 80.37) (width 0.2) (layer "F.Cu") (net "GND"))
 (segment (start 113.8295 101.08825) (end 115.62983 99.28792) (width 0.2) (layer "F.Cu") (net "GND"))
 (segment (start 123.37 80.37) (end 117.986641 85.753359) (width 0.2) (layer "F.Cu") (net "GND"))
 (segment (start 102.04 65.92) (end 122.46 65.92) (width 0.2) (layer "F.Cu") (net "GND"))
 (segment (start 140.682 75.5) (end 156.19 59.992) (width 0.2) (layer "F.Cu") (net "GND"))
 (segment (start 119.573532 102.10025) (end 116.195516 98.722234) (width 0.2) (layer "F.Cu") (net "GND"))
 (segment (start 123.37 80.37) (end 123.37 74.45) (width 0.2) (layer "F.Cu") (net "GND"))
 (segment (start 123.37 74.45) (end 130.99 74.45) (width 0.2) (layer "F.Cu") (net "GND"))
 (segment (start 122.46 65.92) (end 132.04 75.5) (width 0.2) (layer "F.Cu") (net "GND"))
 (segment (start 117.986641 85.753359) (end 117.986641 99.417391) (width 0.2) (layer "F.Cu") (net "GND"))
 (segment (start 155.92 103.5) (end 146.5 103.5) (width 0.2) (layer "F.Cu") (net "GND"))
 (segment (start 130.99 74.45) (end 132.04 75.5) (width 0.2) (layer "F.Cu") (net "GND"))
 (segment (start 159 100.42) (end 155.92 103.5) (width 0.2) (layer "F.Cu") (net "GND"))
 (segment (start 104.5045 102.10025) (end 92.82 90.41575) (width 0.2) (layer "F.Cu") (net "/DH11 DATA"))
 (segment (start 133.81 62) (end 133.5 62) (width 0.2) (layer "F.Cu") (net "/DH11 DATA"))
 (segment (start 92.82 90.41575) (end 92.82 68.218729) (width 0.2) (layer "F.Cu") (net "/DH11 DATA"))
 (segment (start 103.66173 57.377) (end 126.96 57.377) (width 0.2) (layer "F.Cu") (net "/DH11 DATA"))
 (segment (start 131 59.5) (end 136 59.5) (width 0.2) (layer "F.Cu") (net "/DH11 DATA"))
 (segment (start 133.5 62) (end 131 59.5) (width 0.2) (layer "F.Cu") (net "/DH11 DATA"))
 (segment (start 133.81 68.65) (end 129.782843 72.677157) (width 0.2) (layer "F.Cu") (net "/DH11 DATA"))
 (segment (start 92.82 68.218729) (end 103.66173 57.377) (width 0.2) (layer "F.Cu") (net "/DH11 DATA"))
 (segment (start 133.81 62) (end 133.81 68.65) (width 0.2) (layer "F.Cu") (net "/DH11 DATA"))
 (segment (start 104.5045 104.64025) (end 102.8295 106.31525) (width 0.2) (layer "F.Cu") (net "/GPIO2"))
 (segment (start 104.090858 116.90025) (end 140.15 116.90025) (width 0.2) (layer "F.Cu") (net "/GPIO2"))
 (segment (start 102.8295 115.638892) (end 104.090858 116.90025) (width 0.2) (layer "F.Cu") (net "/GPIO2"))
 (segment (start 102.8295 106.31525) (end 102.8295 115.638892) (width 0.2) (layer "F.Cu") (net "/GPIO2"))
 (segment (start 96.75 69.52) (end 96.75 88.726422) (width 0.2) (layer "F.Cu") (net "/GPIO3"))
 (segment (start 96.75 88.726422) (end 109.6645 101.640922) (width 0.2) (layer "F.Cu") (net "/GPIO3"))
 (segment (start 109.6645 105.414042) (end 109.335292 105.74325) (width 0.2) (layer "F.Cu") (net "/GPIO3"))
 (segment (start 105.9415 105.74325) (end 104.5045 107.18025) (width 0.2) (layer "F.Cu") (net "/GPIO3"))
 (segment (start 109.335292 105.74325) (end 105.9415 105.74325) (width 0.2) (layer "F.Cu") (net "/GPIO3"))
 (segment (start 95.69 68.46) (end 96.75 69.52) (width 0.2) (layer "F.Cu") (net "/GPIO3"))
 (segment (start 109.6645 101.640922) (end 109.6645 105.414042) (width 0.2) (layer "F.Cu") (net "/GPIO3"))
 (segment (start 93.22 68.384415) (end 93.22 88.27575) (width 0.2) (layer "F.Cu") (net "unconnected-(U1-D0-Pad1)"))
 (segment (start 160.681346 57.777) (end 103.827415 57.777) (width 0.2) (layer "F.Cu") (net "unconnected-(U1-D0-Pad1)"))
 (segment (start 162.42 59.515654) (end 162.42 82.75) (width 0.2) (layer "F.Cu") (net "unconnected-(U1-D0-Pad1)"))
 (segment (start 161.67 83.5) (end 161.67 87.5) (width 0.2) (layer "F.Cu") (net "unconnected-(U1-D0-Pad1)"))
 (segment (start 103.827415 57.777) (end 93.22 68.384415) (width 0.2) (layer "F.Cu") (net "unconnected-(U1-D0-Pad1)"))
 (segment (start 162.42 59.515654) (end 160.681346 57.777) (width 0.2) (layer "F.Cu") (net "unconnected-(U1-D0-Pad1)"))
 (segment (start 161.67 87.5) (end 162.42 86.75) (width 0.2) (layer "F.Cu") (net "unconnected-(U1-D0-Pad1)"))
 (segment (start 162.42 82.75) (end 161.67 83.5) (width 0.2) (layer "F.Cu") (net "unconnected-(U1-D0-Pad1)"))
 (segment (start 162.42 86.75) (end 162.42 59.515654) (width 0.2) (layer "F.Cu") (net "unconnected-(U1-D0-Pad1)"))
 (segment (start 93.22 88.27575) (end 104.5045 99.56025) (width 0.2) (layer "F.Cu") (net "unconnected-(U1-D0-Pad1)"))
 (segment (start 158.541346 58.177) (end 159.88 59.515654) (width 0.2) (layer "F.Cu") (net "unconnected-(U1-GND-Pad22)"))
 (segment (start 141.089899 105) (end 140.729899 104.64) (width 0.2) (layer "F.Cu") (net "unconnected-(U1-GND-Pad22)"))
 (segment (start 103.993101 58.177) (end 158.541346 58.177) (width 0.2) (layer "F.Cu") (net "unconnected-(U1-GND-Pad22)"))
 (segment (start 158.523654 101.57) (end 155.093654 105) (width 0.2) (layer "F.Cu") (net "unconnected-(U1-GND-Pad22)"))
 (segment (start 160.15 100.896346) (end 159.476346 101.57) (width 0.2) (layer "F.Cu") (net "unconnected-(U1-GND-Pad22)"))
 (segment (start 159.88 59.515654) (end 159.88 60.468346) (width 0.2) (layer "F.Cu") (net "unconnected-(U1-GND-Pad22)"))
 (segment (start 140.729899 104.64) (end 139.570101 104.64) (width 0.2) (layer "F.Cu") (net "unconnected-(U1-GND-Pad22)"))
 (segment (start 139.570101 104.64) (end 138.75 105.460101) (width 0.2) (layer "F.Cu") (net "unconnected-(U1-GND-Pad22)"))
 (segment (start 160.15 60.738346) (end 160.15 100.896346) (width 0.2) (layer "F.Cu") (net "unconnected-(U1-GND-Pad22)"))
 (segment (start 155.093654 105) (end 141.089899 105) (width 0.2) (layer "F.Cu") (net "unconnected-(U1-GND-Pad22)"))
 (segment (start 96.269899 71.019798) (end 94.29 69.039899) (width 0.2) (layer "F.Cu") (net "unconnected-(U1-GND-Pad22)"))
 (segment (start 159.476346 101.57) (end 158.523654 101.57) (width 0.2) (layer "F.Cu") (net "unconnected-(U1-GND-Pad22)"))
 (segment (start 159.88 60.468346) (end 160.15 60.738346) (width 0.2) (layer "F.Cu") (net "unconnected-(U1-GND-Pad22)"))
 (segment (start 94.29 69.039899) (end 94.29 67.880101) (width 0.2) (layer "F.Cu") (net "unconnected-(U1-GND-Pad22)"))
 (segment (start 108.1145 104.89325) (end 108.1145 100.656608) (width 0.2) (layer "F.Cu") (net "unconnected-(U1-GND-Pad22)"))
 (segment (start 96.269899 88.812007) (end 96.269899 71.019798) (width 0.2) (layer "F.Cu") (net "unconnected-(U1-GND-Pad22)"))
 (segment (start 94.29 67.880101) (end 103.993101 58.177) (width 0.2) (layer "F.Cu") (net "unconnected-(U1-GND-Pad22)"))
 (segment (start 108.1145 100.656608) (end 96.269899 88.812007) (width 0.2) (layer "F.Cu") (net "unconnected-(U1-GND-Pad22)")))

